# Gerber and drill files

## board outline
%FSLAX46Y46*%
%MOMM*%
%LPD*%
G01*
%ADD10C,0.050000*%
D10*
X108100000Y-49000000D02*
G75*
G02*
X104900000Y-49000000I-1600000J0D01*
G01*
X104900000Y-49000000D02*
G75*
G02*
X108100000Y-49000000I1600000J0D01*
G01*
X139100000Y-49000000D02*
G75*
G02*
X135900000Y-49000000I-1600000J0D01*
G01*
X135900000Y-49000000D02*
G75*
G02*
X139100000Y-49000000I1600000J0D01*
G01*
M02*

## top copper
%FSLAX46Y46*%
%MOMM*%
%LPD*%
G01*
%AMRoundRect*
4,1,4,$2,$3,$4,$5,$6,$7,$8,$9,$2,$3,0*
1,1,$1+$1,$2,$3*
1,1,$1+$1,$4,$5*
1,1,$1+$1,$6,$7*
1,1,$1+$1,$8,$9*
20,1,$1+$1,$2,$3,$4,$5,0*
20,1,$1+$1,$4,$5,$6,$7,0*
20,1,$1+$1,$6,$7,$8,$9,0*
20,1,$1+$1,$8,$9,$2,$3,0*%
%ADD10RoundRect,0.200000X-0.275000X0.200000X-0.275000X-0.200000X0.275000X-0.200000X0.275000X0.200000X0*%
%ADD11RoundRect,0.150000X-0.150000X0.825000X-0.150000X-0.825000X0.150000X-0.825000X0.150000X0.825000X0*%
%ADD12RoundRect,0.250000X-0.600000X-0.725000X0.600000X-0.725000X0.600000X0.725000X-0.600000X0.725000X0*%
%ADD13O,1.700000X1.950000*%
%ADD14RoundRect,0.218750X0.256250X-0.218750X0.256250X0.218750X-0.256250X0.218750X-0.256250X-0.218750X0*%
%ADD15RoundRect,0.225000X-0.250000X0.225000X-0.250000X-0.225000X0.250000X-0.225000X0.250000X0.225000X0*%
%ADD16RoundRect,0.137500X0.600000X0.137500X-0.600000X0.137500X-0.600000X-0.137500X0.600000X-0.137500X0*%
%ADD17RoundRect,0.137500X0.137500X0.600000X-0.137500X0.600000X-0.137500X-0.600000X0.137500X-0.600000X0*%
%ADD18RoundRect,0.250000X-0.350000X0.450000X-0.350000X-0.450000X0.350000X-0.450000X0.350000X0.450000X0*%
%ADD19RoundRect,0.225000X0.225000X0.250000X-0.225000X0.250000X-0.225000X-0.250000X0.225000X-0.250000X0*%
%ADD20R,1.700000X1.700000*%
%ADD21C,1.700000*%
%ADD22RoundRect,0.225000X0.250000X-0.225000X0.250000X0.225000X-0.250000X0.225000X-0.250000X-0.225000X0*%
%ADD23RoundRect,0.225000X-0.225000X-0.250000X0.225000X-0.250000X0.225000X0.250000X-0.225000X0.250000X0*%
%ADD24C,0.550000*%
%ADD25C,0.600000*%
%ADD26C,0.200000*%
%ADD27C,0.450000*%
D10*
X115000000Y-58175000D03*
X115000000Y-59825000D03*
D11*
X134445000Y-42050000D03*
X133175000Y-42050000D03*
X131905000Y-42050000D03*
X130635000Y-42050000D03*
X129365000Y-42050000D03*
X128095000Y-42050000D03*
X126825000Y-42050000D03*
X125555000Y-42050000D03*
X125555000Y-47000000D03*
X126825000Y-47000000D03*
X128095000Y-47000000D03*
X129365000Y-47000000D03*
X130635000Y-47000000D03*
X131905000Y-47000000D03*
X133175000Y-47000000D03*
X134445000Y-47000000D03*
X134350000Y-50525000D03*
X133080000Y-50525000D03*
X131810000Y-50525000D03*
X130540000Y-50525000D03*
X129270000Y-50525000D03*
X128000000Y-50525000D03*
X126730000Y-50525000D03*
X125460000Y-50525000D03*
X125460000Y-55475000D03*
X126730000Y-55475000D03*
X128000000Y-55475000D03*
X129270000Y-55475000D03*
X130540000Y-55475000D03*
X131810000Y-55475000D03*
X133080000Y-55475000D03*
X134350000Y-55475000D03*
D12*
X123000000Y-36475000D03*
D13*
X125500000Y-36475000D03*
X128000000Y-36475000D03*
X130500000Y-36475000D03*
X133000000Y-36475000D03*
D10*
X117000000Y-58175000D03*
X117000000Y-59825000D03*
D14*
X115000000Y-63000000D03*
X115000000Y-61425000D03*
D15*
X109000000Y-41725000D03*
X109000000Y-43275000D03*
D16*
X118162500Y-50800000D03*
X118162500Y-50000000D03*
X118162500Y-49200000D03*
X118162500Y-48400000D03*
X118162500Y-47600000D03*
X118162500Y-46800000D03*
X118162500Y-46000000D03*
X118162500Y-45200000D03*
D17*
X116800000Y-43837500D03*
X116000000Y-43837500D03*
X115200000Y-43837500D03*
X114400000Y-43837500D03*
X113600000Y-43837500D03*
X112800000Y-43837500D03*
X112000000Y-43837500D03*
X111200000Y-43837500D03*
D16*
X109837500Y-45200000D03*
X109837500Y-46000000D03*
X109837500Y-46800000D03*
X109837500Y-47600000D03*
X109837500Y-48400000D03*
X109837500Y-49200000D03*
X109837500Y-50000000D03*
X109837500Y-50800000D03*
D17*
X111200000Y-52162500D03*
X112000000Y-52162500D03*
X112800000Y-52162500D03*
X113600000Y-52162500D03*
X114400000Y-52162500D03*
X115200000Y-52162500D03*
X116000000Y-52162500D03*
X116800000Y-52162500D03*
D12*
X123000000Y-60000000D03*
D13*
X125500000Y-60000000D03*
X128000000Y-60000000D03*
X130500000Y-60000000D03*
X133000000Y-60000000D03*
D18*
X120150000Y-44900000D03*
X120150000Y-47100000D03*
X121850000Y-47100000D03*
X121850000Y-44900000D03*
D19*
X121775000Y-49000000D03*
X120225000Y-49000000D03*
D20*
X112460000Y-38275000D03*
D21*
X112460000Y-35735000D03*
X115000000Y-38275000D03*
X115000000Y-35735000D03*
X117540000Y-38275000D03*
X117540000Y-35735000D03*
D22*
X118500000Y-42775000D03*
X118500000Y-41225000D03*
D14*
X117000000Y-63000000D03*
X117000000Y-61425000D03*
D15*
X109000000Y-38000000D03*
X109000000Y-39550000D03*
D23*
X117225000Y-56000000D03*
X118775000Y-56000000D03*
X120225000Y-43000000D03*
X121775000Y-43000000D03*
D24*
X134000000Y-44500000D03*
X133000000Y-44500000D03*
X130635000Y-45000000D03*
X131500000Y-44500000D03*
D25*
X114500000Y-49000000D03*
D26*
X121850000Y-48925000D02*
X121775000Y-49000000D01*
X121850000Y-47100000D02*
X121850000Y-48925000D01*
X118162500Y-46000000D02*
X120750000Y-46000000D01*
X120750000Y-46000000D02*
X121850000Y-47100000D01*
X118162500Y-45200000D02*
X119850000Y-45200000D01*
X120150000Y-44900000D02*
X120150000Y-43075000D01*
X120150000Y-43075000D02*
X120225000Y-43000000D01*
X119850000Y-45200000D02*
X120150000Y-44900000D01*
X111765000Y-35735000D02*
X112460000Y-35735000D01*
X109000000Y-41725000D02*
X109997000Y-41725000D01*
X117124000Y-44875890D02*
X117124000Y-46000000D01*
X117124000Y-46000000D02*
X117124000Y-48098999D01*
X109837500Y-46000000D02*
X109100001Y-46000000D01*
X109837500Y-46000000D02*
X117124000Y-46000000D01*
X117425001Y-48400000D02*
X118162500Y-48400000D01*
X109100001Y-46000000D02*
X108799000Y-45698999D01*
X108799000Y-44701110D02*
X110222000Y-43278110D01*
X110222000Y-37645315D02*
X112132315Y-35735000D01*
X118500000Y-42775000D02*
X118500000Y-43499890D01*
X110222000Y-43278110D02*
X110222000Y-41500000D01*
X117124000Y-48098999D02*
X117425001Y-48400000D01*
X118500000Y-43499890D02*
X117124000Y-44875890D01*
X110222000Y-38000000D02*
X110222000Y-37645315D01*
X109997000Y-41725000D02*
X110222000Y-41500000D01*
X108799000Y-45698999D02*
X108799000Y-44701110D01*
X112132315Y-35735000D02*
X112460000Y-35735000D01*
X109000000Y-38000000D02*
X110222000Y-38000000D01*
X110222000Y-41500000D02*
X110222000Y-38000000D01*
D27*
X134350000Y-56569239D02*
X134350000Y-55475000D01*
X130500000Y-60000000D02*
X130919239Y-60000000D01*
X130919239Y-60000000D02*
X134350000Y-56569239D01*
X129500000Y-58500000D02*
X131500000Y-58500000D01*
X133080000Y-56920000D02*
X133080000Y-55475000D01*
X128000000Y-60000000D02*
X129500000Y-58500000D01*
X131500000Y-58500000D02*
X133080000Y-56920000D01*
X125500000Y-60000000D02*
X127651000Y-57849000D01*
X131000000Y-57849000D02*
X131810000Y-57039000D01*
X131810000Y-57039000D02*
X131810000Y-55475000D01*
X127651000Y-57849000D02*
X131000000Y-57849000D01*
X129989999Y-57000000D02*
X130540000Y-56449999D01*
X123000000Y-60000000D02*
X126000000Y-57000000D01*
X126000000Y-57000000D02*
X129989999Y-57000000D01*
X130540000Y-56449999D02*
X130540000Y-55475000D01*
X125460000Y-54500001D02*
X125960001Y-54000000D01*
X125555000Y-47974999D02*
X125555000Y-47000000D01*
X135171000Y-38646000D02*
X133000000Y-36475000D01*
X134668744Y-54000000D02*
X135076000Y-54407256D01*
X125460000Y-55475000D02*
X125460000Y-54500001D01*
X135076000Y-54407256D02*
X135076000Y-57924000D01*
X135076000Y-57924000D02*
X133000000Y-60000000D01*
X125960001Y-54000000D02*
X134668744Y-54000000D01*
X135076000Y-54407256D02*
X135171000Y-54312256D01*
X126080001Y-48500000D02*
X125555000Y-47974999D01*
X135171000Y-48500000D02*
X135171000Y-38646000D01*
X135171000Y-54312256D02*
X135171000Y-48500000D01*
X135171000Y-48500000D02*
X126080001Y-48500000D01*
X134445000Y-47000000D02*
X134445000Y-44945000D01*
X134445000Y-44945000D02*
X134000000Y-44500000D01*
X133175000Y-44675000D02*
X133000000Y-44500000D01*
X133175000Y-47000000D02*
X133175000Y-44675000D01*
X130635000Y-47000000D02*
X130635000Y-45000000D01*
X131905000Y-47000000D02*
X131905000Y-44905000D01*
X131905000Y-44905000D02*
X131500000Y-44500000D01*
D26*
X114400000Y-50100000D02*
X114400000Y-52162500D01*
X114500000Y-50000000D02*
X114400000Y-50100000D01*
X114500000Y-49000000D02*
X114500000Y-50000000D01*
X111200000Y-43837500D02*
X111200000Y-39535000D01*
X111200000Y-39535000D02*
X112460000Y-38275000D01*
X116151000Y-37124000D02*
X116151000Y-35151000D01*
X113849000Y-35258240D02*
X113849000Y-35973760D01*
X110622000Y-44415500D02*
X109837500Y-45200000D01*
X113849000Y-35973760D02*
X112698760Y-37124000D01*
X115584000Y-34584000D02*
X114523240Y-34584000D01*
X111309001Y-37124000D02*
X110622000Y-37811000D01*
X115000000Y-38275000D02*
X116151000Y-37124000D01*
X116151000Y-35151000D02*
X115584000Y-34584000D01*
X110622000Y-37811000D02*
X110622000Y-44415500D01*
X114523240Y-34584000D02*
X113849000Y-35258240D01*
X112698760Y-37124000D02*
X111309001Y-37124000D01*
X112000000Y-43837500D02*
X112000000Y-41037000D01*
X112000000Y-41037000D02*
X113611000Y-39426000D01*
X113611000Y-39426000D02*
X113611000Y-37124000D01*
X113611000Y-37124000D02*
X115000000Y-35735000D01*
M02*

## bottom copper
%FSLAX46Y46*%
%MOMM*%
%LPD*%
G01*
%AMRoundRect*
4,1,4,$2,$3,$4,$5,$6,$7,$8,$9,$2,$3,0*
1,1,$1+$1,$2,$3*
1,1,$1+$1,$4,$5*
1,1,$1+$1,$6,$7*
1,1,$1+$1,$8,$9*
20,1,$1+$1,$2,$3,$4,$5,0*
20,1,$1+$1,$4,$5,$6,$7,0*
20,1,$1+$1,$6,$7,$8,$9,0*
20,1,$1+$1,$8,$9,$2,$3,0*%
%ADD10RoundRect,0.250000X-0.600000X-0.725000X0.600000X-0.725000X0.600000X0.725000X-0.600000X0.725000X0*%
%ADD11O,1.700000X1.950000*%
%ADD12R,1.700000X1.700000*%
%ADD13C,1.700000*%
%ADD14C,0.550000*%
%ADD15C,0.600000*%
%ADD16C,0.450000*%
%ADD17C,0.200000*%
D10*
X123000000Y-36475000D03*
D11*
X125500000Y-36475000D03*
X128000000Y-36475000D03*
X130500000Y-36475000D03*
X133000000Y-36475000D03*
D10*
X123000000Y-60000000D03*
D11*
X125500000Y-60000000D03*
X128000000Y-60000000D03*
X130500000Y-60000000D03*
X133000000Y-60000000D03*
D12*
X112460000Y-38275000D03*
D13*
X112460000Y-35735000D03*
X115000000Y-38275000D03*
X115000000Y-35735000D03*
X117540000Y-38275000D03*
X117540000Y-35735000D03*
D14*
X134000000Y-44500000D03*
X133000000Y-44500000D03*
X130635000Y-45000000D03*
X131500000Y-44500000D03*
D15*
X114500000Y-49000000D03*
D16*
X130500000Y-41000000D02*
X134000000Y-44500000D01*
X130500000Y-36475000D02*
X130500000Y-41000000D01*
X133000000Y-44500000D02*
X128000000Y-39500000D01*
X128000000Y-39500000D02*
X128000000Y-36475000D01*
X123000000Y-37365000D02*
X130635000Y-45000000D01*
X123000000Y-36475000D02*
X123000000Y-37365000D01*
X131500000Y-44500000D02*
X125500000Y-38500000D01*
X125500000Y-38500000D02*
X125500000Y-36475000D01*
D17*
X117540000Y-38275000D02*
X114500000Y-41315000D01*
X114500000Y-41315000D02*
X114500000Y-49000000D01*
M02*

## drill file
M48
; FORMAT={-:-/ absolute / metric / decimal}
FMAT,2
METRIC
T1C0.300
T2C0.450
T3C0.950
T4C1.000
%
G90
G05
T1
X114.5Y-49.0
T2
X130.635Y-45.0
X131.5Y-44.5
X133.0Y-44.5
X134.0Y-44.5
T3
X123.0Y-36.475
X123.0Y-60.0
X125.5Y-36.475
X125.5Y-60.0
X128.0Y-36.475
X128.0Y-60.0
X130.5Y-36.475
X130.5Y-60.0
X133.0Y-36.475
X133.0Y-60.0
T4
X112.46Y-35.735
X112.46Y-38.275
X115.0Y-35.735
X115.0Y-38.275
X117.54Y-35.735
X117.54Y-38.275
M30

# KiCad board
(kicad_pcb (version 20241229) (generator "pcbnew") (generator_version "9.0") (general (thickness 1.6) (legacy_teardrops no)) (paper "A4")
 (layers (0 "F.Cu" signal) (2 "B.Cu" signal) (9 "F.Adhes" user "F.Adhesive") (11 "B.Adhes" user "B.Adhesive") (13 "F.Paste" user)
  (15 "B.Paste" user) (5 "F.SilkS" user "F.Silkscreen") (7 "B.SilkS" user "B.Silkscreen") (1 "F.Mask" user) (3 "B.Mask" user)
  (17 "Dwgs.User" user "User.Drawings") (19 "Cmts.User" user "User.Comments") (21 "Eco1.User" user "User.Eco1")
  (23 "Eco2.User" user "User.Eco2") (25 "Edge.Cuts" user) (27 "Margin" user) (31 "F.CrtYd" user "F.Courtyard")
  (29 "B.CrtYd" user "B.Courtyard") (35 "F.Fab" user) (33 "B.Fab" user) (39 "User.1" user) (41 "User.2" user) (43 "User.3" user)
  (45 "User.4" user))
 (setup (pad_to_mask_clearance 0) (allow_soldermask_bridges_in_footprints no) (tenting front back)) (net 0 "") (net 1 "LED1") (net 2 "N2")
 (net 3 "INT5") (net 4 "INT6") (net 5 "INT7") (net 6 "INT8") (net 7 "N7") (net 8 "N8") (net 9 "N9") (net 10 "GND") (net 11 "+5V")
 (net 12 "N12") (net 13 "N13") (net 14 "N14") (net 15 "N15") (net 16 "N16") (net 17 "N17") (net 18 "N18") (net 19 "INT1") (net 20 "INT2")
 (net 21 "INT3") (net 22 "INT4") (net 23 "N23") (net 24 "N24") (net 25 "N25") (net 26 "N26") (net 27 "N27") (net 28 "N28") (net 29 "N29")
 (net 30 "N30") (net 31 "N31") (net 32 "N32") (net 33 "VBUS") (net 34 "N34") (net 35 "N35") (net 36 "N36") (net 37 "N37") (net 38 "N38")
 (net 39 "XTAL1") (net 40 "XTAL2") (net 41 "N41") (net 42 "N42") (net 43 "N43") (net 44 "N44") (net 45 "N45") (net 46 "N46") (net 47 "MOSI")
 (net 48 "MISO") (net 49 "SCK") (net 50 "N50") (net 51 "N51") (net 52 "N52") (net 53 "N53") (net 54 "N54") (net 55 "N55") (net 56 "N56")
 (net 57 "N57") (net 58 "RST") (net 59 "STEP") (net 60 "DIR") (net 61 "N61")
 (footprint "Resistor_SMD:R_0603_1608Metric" (layer "F.Cu") (at 115 59 -90)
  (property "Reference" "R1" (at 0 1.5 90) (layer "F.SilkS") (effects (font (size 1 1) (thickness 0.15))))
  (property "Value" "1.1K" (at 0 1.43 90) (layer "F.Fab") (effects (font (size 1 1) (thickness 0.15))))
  (pad "1" smd roundrect (at -0.825 0 270) (size 0.8 0.95) (layers "F.Cu" "F.Mask" "F.Paste") (roundrect_rratio 0.25) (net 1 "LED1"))
  (pad "2" smd roundrect (at 0.825 0 270) (size 0.8 0.95) (layers "F.Cu" "F.Mask" "F.Paste") (roundrect_rratio 0.25) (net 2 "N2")))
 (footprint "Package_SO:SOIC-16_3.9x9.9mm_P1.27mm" (layer "F.Cu") (at 130 44.525 -90)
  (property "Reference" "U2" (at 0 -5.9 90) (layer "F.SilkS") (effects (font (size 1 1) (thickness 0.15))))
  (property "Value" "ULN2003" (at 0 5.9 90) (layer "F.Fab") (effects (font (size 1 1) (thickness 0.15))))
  (pad "1" smd roundrect (at -2.475 -4.445 270) (size 1.95 0.6) (layers "F.Cu" "F.Mask" "F.Paste") (roundrect_rratio 0.25) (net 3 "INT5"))
  (pad "2" smd roundrect (at -2.475 -3.175 270) (size 1.95 0.6) (layers "F.Cu" "F.Mask" "F.Paste") (roundrect_rratio 0.25) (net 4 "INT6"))
  (pad "3" smd roundrect (at -2.475 -1.905 270) (size 1.95 0.6) (layers "F.Cu" "F.Mask" "F.Paste") (roundrect_rratio 0.25) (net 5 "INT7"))
  (pad "4" smd roundrect (at -2.475 -0.635 270) (size 1.95 0.6) (layers "F.Cu" "F.Mask" "F.Paste") (roundrect_rratio 0.25) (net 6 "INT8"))
  (pad "5" smd roundrect (at -2.475 0.635 270) (size 1.95 0.6) (layers "F.Cu" "F.Mask" "F.Paste") (roundrect_rratio 0.25) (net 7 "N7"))
  (pad "6" smd roundrect (at -2.475 1.905 270) (size 1.95 0.6) (layers "F.Cu" "F.Mask" "F.Paste") (roundrect_rratio 0.25) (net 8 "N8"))
  (pad "7" smd roundrect (at -2.475 3.175 270) (size 1.95 0.6) (layers "F.Cu" "F.Mask" "F.Paste") (roundrect_rratio 0.25) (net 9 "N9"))
  (pad "8" smd roundrect (at -2.475 4.445 270) (size 1.95 0.6) (layers "F.Cu" "F.Mask" "F.Paste") (roundrect_rratio 0.25) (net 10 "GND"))
  (pad "9" smd roundrect (at 2.475 4.445 270) (size 1.95 0.6) (layers "F.Cu" "F.Mask" "F.Paste") (roundrect_rratio 0.25) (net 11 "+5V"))
  (pad "10" smd roundrect (at 2.475 3.175 270) (size 1.95 0.6) (layers "F.Cu" "F.Mask" "F.Paste") (roundrect_rratio 0.25) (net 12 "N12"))
  (pad "11" smd roundrect (at 2.475 1.905 270) (size 1.95 0.6) (layers "F.Cu" "F.Mask" "F.Paste") (roundrect_rratio 0.25) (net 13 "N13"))
  (pad "12" smd roundrect (at 2.475 0.635 270) (size 1.95 0.6) (layers "F.Cu" "F.Mask" "F.Paste") (roundrect_rratio 0.25) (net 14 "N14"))
  (pad "13" smd roundrect (at 2.475 -0.635 270) (size 1.95 0.6) (layers "F.Cu" "F.Mask" "F.Paste") (roundrect_rratio 0.25) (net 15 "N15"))
  (pad "14" smd roundrect (at 2.475 -1.905 270) (size 1.95 0.6) (layers "F.Cu" "F.Mask" "F.Paste") (roundrect_rratio 0.25) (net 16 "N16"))
  (pad "15" smd roundrect (at 2.475 -3.175 270) (size 1.95 0.6) (layers "F.Cu" "F.Mask" "F.Paste") (roundrect_rratio 0.25) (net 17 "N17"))
  (pad "16" smd roundrect (at 2.475 -4.445 270) (size 1.95 0.6) (layers "F.Cu" "F.Mask" "F.Paste") (roundrect_rratio 0.25) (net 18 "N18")))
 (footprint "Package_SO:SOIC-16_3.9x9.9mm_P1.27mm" (layer "F.Cu") (at 129.905 53 -90)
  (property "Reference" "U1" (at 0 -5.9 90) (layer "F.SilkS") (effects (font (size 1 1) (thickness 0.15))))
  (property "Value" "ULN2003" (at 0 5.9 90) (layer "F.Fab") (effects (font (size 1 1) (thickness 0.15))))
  (pad "1" smd roundrect (at -2.475 -4.445 270) (size 1.95 0.6) (layers "F.Cu" "F.Mask" "F.Paste") (roundrect_rratio 0.25) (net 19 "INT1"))
  (pad "2" smd roundrect (at -2.475 -3.175 270) (size 1.95 0.6) (layers "F.Cu" "F.Mask" "F.Paste") (roundrect_rratio 0.25) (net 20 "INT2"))
  (pad "3" smd roundrect (at -2.475 -1.905 270) (size 1.95 0.6) (layers "F.Cu" "F.Mask" "F.Paste") (roundrect_rratio 0.25) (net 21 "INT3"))
  (pad "4" smd roundrect (at -2.475 -0.635 270) (size 1.95 0.6) (layers "F.Cu" "F.Mask" "F.Paste") (roundrect_rratio 0.25) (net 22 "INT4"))
  (pad "5" smd roundrect (at -2.475 0.635 270) (size 1.95 0.6) (layers "F.Cu" "F.Mask" "F.Paste") (roundrect_rratio 0.25) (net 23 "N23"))
  (pad "6" smd roundrect (at -2.475 1.905 270) (size 1.95 0.6) (layers "F.Cu" "F.Mask" "F.Paste") (roundrect_rratio 0.25) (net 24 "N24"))
  (pad "7" smd roundrect (at -2.475 3.175 270) (size 1.95 0.6) (layers "F.Cu" "F.Mask" "F.Paste") (roundrect_rratio 0.25) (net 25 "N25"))
  (pad "8" smd roundrect (at -2.475 4.445 270) (size 1.95 0.6) (layers "F.Cu" "F.Mask" "F.Paste") (roundrect_rratio 0.25) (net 10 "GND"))
  (pad "9" smd roundrect (at 2.475 4.445 270) (size 1.95 0.6) (layers "F.Cu" "F.Mask" "F.Paste") (roundrect_rratio 0.25) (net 11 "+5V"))
  (pad "10" smd roundrect (at 2.475 3.175 270) (size 1.95 0.6) (layers "F.Cu" "F.Mask" "F.Paste") (roundrect_rratio 0.25) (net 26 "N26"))
  (pad "11" smd roundrect (at 2.475 1.905 270) (size 1.95 0.6) (layers "F.Cu" "F.Mask" "F.Paste") (roundrect_rratio 0.25) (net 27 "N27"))
  (pad "12" smd roundrect (at 2.475 0.635 270) (size 1.95 0.6) (layers "F.Cu" "F.Mask" "F.Paste") (roundrect_rratio 0.25) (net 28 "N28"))
  (pad "13" smd roundrect (at 2.475 -0.635 270) (size 1.95 0.6) (layers "F.Cu" "F.Mask" "F.Paste") (roundrect_rratio 0.25) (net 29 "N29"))
  (pad "14" smd roundrect (at 2.475 -1.905 270) (size 1.95 0.6) (layers "F.Cu" "F.Mask" "F.Paste") (roundrect_rratio 0.25) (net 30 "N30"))
  (pad "15" smd roundrect (at 2.475 -3.175 270) (size 1.95 0.6) (layers "F.Cu" "F.Mask" "F.Paste") (roundrect_rratio 0.25) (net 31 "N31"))
  (pad "16" smd roundrect (at 2.475 -4.445 270) (size 1.95 0.6) (layers "F.Cu" "F.Mask" "F.Paste") (roundrect_rratio 0.25) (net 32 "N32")))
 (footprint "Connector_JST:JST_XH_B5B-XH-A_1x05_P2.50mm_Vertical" (layer "F.Cu") (at 123 36.475)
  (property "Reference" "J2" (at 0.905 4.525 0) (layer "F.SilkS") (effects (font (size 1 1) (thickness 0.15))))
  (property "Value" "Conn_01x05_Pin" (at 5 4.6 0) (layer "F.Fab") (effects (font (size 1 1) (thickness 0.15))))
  (pad "1" thru_hole roundrect (at 0 0) (size 1.7 1.95) (drill 0.95) (layers "*.Cu" "*.Mask") (remove_unused_layers no)
   (roundrect_rratio 0.147059) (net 15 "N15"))
  (pad "2" thru_hole oval (at 2.5 0) (size 1.7 1.95) (drill 0.95) (layers "*.Cu" "*.Mask") (remove_unused_layers no) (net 16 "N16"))
  (pad "3" thru_hole oval (at 5 0) (size 1.7 1.95) (drill 0.95) (layers "*.Cu" "*.Mask") (remove_unused_layers no) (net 17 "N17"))
  (pad "4" thru_hole oval (at 7.5 0) (size 1.7 1.95) (drill 0.95) (layers "*.Cu" "*.Mask") (remove_unused_layers no) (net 18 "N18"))
  (pad "5" thru_hole oval (at 10 0) (size 1.7 1.95) (drill 0.95) (layers "*.Cu" "*.Mask") (remove_unused_layers no) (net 11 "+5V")))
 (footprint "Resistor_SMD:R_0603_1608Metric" (layer "F.Cu") (at 117 59 -90)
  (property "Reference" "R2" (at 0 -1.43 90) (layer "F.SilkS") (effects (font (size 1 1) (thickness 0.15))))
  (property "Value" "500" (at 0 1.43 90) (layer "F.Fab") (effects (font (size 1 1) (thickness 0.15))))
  (pad "1" smd roundrect (at -0.825 0 270) (size 0.8 0.95) (layers "F.Cu" "F.Mask" "F.Paste") (roundrect_rratio 0.25) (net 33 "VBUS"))
  (pad "2" smd roundrect (at 0.825 0 270) (size 0.8 0.95) (layers "F.Cu" "F.Mask" "F.Paste") (roundrect_rratio 0.25) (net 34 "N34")))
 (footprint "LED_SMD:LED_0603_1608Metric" (layer "F.Cu") (at 115 62.2125 90)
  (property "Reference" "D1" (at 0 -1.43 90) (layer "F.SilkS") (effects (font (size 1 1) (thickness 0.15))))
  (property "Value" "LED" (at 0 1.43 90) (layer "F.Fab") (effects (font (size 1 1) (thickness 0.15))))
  (pad "1" smd roundrect (at -0.7875 0 90) (size 0.875 0.95) (layers "F.Cu" "F.Mask" "F.Paste") (roundrect_rratio 0.25) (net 10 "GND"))
  (pad "2" smd roundrect (at 0.7875 0 90) (size 0.875 0.95) (layers "F.Cu" "F.Mask" "F.Paste") (roundrect_rratio 0.25) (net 2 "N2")))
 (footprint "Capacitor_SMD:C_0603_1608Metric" (layer "F.Cu") (at 109 42.5 -90)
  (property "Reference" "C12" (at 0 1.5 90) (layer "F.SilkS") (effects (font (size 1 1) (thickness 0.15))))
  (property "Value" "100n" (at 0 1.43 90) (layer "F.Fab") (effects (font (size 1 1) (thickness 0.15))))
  (pad "1" smd roundrect (at -0.775 0 270) (size 0.9 0.95) (layers "F.Cu" "F.Mask" "F.Paste") (roundrect_rratio 0.25) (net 33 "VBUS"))
  (pad "2" smd roundrect (at 0.775 0 270) (size 0.9 0.95) (layers "F.Cu" "F.Mask" "F.Paste") (roundrect_rratio 0.25) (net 10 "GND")))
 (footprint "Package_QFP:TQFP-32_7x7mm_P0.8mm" (layer "F.Cu") (at 114 48 180)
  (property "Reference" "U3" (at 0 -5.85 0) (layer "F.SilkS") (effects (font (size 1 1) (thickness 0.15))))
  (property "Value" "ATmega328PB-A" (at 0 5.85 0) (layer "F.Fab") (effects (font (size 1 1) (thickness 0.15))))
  (pad "1" smd roundrect (at -4.1625 -2.8 180) (size 1.475 0.55) (layers "F.Cu" "F.Mask" "F.Paste") (roundrect_rratio 0.25) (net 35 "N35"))
  (pad "2" smd roundrect (at -4.1625 -2 180) (size 1.475 0.55) (layers "F.Cu" "F.Mask" "F.Paste") (roundrect_rratio 0.25) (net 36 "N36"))
  (pad "3" smd roundrect (at -4.1625 -1.2 180) (size 1.475 0.55) (layers "F.Cu" "F.Mask" "F.Paste") (roundrect_rratio 0.25) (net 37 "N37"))
  (pad "4" smd roundrect (at -4.1625 -0.4 180) (size 1.475 0.55) (layers "F.Cu" "F.Mask" "F.Paste") (roundrect_rratio 0.25) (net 33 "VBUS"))
  (pad "5" smd roundrect (at -4.1625 0.4 180) (size 1.475 0.55) (layers "F.Cu" "F.Mask" "F.Paste") (roundrect_rratio 0.25) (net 10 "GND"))
  (pad "6" smd roundrect (at -4.1625 1.2 180) (size 1.475 0.55) (layers "F.Cu" "F.Mask" "F.Paste") (roundrect_rratio 0.25) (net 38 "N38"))
  (pad "7" smd roundrect (at -4.1625 2 180) (size 1.475 0.55) (layers "F.Cu" "F.Mask" "F.Paste") (roundrect_rratio 0.25) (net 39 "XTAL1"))
  (pad "8" smd roundrect (at -4.1625 2.8 180) (size 1.475 0.55) (layers "F.Cu" "F.Mask" "F.Paste") (roundrect_rratio 0.25) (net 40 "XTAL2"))
  (pad "9" smd roundrect (at -2.8 4.1625 180) (size 0.55 1.475) (layers "F.Cu" "F.Mask" "F.Paste") (roundrect_rratio 0.25) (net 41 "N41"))
  (pad "10" smd roundrect (at -2 4.1625 180) (size 0.55 1.475) (layers "F.Cu" "F.Mask" "F.Paste") (roundrect_rratio 0.25) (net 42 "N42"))
  (pad "11" smd roundrect (at -1.2 4.1625 180) (size 0.55 1.475) (layers "F.Cu" "F.Mask" "F.Paste") (roundrect_rratio 0.25) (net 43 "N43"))
  (pad "12" smd roundrect (at -0.4 4.1625 180) (size 0.55 1.475) (layers "F.Cu" "F.Mask" "F.Paste") (roundrect_rratio 0.25) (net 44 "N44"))
  (pad "13" smd roundrect (at 0.4 4.1625 180) (size 0.55 1.475) (layers "F.Cu" "F.Mask" "F.Paste") (roundrect_rratio 0.25) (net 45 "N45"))
  (pad "14" smd roundrect (at 1.2 4.1625 180) (size 0.55 1.475) (layers "F.Cu" "F.Mask" "F.Paste") (roundrect_rratio 0.25) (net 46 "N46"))
  (pad "15" smd roundrect (at 2 4.1625 180) (size 0.55 1.475) (layers "F.Cu" "F.Mask" "F.Paste") (roundrect_rratio 0.25) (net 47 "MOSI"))
  (pad "16" smd roundrect (at 2.8 4.1625 180) (size 0.55 1.475) (layers "F.Cu" "F.Mask" "F.Paste") (roundrect_rratio 0.25) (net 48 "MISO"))
  (pad "17" smd roundrect (at 4.1625 2.8 180) (size 1.475 0.55) (layers "F.Cu" "F.Mask" "F.Paste") (roundrect_rratio 0.25) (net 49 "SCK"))
  (pad "18" smd roundrect (at 4.1625 2 180) (size 1.475 0.55) (layers "F.Cu" "F.Mask" "F.Paste") (roundrect_rratio 0.25) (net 33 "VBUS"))
  (pad "19" smd roundrect (at 4.1625 1.2 180) (size 1.475 0.55) (layers "F.Cu" "F.Mask" "F.Paste") (roundrect_rratio 0.25) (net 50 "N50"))
  (pad "20" smd roundrect (at 4.1625 0.4 180) (size 1.475 0.55) (layers "F.Cu" "F.Mask" "F.Paste") (roundrect_rratio 0.25) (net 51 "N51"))
  (pad "21" smd roundrect (at 4.1625 -0.4 180) (size 1.475 0.55) (layers "F.Cu" "F.Mask" "F.Paste") (roundrect_rratio 0.25) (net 10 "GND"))
  (pad "22" smd roundrect (at 4.1625 -1.2 180) (size 1.475 0.55) (layers "F.Cu" "F.Mask" "F.Paste") (roundrect_rratio 0.25) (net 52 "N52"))
  (pad "23" smd roundrect (at 4.1625 -2 180) (size 1.475 0.55) (layers "F.Cu" "F.Mask" "F.Paste") (roundrect_rratio 0.25) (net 1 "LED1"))
  (pad "24" smd roundrect (at 4.1625 -2.8 180) (size 1.475 0.55) (layers "F.Cu" "F.Mask" "F.Paste") (roundrect_rratio 0.25) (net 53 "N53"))
  (pad "25" smd roundrect (at 2.8 -4.1625 180) (size 0.55 1.475) (layers "F.Cu" "F.Mask" "F.Paste") (roundrect_rratio 0.25) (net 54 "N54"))
  (pad "26" smd roundrect (at 2 -4.1625 180) (size 0.55 1.475) (layers "F.Cu" "F.Mask" "F.Paste") (roundrect_rratio 0.25) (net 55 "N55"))
  (pad "27" smd roundrect (at 1.2 -4.1625 180) (size 0.55 1.475) (layers "F.Cu" "F.Mask" "F.Paste") (roundrect_rratio 0.25) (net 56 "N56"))
  (pad "28" smd roundrect (at 0.4 -4.1625 180) (size 0.55 1.475) (layers "F.Cu" "F.Mask" "F.Paste") (roundrect_rratio 0.25) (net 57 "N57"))
  (pad "29" smd roundrect (at -0.4 -4.1625 180) (size 0.55 1.475) (layers "F.Cu" "F.Mask" "F.Paste") (roundrect_rratio 0.25) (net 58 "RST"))
  (pad "30" smd roundrect (at -1.2 -4.1625 180) (size 0.55 1.475) (layers "F.Cu" "F.Mask" "F.Paste") (roundrect_rratio 0.25) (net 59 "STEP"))
  (pad "31" smd roundrect (at -2 -4.1625 180) (size 0.55 1.475) (layers "F.Cu" "F.Mask" "F.Paste") (roundrect_rratio 0.25) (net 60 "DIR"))
  (pad "32" smd roundrect (at -2.8 -4.1625 180) (size 0.55 1.475) (layers "F.Cu" "F.Mask" "F.Paste") (roundrect_rratio 0.25) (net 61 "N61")))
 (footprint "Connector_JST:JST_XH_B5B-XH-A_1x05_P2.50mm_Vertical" (layer "F.Cu") (at 123 60)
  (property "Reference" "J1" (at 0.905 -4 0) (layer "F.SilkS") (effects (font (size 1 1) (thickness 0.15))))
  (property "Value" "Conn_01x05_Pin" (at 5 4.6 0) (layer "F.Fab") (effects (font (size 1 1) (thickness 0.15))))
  (pad "1" thru_hole roundrect (at 0 0) (size 1.7 1.95) (drill 0.95) (layers "*.Cu" "*.Mask") (remove_unused_layers no)
   (roundrect_rratio 0.147059) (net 29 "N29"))
  (pad "2" thru_hole oval (at 2.5 0) (size 1.7 1.95) (drill 0.95) (layers "*.Cu" "*.Mask") (remove_unused_layers no) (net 30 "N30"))
  (pad "3" thru_hole oval (at 5 0) (size 1.7 1.95) (drill 0.95) (layers "*.Cu" "*.Mask") (remove_unused_layers no) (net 31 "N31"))
  (pad "4" thru_hole oval (at 7.5 0) (size 1.7 1.95) (drill 0.95) (layers "*.Cu" "*.Mask") (remove_unused_layers no) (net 32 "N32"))
  (pad "5" thru_hole oval (at 10 0) (size 1.7 1.95) (drill 0.95) (layers "*.Cu" "*.Mask") (remove_unused_layers no) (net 11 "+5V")))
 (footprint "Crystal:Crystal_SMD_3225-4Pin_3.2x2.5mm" (layer "F.Cu") (at 121 46 -90)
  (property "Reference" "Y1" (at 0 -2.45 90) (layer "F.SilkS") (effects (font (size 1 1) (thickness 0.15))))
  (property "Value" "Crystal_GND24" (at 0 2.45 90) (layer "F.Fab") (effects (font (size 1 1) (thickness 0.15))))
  (pad "1" smd roundrect (at -1.1 0.85 270) (size 1.4 1.2) (layers "F.Cu" "F.Mask" "F.Paste") (roundrect_rratio 0.208333) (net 40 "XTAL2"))
  (pad "2" smd roundrect (at 1.1 0.85 270) (size 1.4 1.2) (layers "F.Cu" "F.Mask" "F.Paste") (roundrect_rratio 0.208333) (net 10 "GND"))
  (pad "3" smd roundrect (at 1.1 -0.85 270) (size 1.4 1.2) (layers "F.Cu" "F.Mask" "F.Paste") (roundrect_rratio 0.208333) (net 39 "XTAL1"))
  (pad "4" smd roundrect (at -1.1 -0.85 270) (size 1.4 1.2) (layers "F.Cu" "F.Mask" "F.Paste") (roundrect_rratio 0.208333) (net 10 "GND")))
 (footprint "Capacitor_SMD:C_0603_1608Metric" (layer "F.Cu") (at 121 49 180)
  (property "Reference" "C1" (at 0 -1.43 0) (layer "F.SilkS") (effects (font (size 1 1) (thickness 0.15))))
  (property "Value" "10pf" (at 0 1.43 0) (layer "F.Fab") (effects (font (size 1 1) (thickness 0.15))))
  (pad "1" smd roundrect (at -0.775 0 180) (size 0.9 0.95) (layers "F.Cu" "F.Mask" "F.Paste") (roundrect_rratio 0.25) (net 39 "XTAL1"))
  (pad "2" smd roundrect (at 0.775 0 180) (size 0.9 0.95) (layers "F.Cu" "F.Mask" "F.Paste") (roundrect_rratio 0.25) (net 10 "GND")))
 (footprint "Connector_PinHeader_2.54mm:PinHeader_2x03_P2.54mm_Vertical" (layer "F.Cu") (at 112.46 38.275 90)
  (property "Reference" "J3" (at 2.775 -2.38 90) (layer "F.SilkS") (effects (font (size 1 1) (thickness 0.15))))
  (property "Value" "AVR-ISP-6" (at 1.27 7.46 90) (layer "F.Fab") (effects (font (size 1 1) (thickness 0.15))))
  (pad "1" thru_hole rect (at 0 0 90) (size 1.7 1.7) (drill 1) (layers "*.Cu" "*.Mask") (remove_unused_layers no) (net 48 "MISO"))
  (pad "2" thru_hole circle (at 2.54 0 90) (size 1.7 1.7) (drill 1) (layers "*.Cu" "*.Mask") (remove_unused_layers no) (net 33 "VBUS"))
  (pad "3" thru_hole circle (at 0 2.54 90) (size 1.7 1.7) (drill 1) (layers "*.Cu" "*.Mask") (remove_unused_layers no) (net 49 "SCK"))
  (pad "4" thru_hole circle (at 2.54 2.54 90) (size 1.7 1.7) (drill 1) (layers "*.Cu" "*.Mask") (remove_unused_layers no) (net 47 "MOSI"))
  (pad "5" thru_hole circle (at 0 5.08 90) (size 1.7 1.7) (drill 1) (layers "*.Cu" "*.Mask") (remove_unused_layers no) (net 58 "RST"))
  (pad "6" thru_hole circle (at 2.54 5.08 90) (size 1.7 1.7) (drill 1) (layers "*.Cu" "*.Mask") (remove_unused_layers no) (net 10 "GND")))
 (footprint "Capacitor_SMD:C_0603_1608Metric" (layer "F.Cu") (at 118.5 42 90)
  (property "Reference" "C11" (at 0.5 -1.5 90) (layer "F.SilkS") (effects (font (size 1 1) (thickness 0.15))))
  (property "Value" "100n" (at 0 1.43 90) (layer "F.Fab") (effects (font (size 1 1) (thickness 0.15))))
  (pad "1" smd roundrect (at -0.775 0 90) (size 0.9 0.95) (layers "F.Cu" "F.Mask" "F.Paste") (roundrect_rratio 0.25) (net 33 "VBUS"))
  (pad "2" smd roundrect (at 0.775 0 90) (size 0.9 0.95) (layers "F.Cu" "F.Mask" "F.Paste") (roundrect_rratio 0.25) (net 10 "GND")))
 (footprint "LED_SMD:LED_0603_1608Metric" (layer "F.Cu") (at 117 62.2125 90)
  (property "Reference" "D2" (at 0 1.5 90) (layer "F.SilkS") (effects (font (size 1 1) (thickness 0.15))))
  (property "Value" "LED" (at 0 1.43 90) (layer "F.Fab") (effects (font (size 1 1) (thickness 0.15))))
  (pad "1" smd roundrect (at -0.7875 0 90) (size 0.875 0.95) (layers "F.Cu" "F.Mask" "F.Paste") (roundrect_rratio 0.25) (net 10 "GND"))
  (pad "2" smd roundrect (at 0.7875 0 90) (size 0.875 0.95) (layers "F.Cu" "F.Mask" "F.Paste") (roundrect_rratio 0.25) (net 34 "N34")))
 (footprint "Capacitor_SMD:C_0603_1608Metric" (layer "F.Cu") (at 109 38.775 -90)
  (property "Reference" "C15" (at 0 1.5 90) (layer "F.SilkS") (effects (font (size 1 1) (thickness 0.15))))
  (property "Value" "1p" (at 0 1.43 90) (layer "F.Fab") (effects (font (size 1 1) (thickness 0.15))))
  (pad "1" smd roundrect (at -0.775 0 270) (size 0.9 0.95) (layers "F.Cu" "F.Mask" "F.Paste") (roundrect_rratio 0.25) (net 33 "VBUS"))
  (pad "2" smd roundrect (at 0.775 0 270) (size 0.9 0.95) (layers "F.Cu" "F.Mask" "F.Paste") (roundrect_rratio 0.25) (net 10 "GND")))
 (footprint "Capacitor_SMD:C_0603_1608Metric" (layer "F.Cu") (at 118 56)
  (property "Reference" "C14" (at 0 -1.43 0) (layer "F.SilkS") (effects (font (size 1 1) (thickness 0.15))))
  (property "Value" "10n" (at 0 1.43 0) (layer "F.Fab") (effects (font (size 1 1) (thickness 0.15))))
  (pad "1" smd roundrect (at -0.775 0) (size 0.9 0.95) (layers "F.Cu" "F.Mask" "F.Paste") (roundrect_rratio 0.25) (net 33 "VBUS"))
  (pad "2" smd roundrect (at 0.775 0) (size 0.9 0.95) (layers "F.Cu" "F.Mask" "F.Paste") (roundrect_rratio 0.25) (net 10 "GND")))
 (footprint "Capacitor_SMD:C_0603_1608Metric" (layer "F.Cu") (at 121 43)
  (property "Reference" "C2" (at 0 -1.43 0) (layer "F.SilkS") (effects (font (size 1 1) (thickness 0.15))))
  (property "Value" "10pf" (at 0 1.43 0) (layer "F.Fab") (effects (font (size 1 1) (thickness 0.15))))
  (pad "1" smd roundrect (at -0.775 0) (size 0.9 0.95) (layers "F.Cu" "F.Mask" "F.Paste") (roundrect_rratio 0.25) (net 40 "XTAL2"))
  (pad "2" smd roundrect (at 0.775 0) (size 0.9 0.95) (layers "F.Cu" "F.Mask" "F.Paste") (roundrect_rratio 0.25) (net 10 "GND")))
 (gr_circle (center 106.5 49) (end 108.1 49) (stroke (width 0.05) (type solid)) (fill no) (layer "Edge.Cuts"))
 (gr_circle (center 137.5 49) (end 139.1 49) (stroke (width 0.05) (type solid)) (fill no) (layer "Edge.Cuts"))
 (segment (start 121.85 48.925) (end 121.775 49) (width 0.2) (layer "F.Cu") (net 39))
 (segment (start 121.85 47.1) (end 121.85 48.925) (width 0.2) (layer "F.Cu") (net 39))
 (segment (start 118.1625 46) (end 120.75 46) (width 0.2) (layer "F.Cu") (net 39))
 (segment (start 120.75 46) (end 121.85 47.1) (width 0.2) (layer "F.Cu") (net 39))
 (segment (start 118.1625 45.2) (end 119.85 45.2) (width 0.2) (layer "F.Cu") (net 40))
 (segment (start 120.15 44.9) (end 120.15 43.075) (width 0.2) (layer "F.Cu") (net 40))
 (segment (start 120.15 43.075) (end 120.225 43) (width 0.2) (layer "F.Cu") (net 40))
 (segment (start 119.85 45.2) (end 120.15 44.9) (width 0.2) (layer "F.Cu") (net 40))
 (segment (start 111.765 35.735) (end 112.46 35.735) (width 0.2) (layer "F.Cu") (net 33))
 (segment (start 109 41.725) (end 109.997 41.725) (width 0.2) (layer "F.Cu") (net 33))
 (segment (start 117.124 44.87589) (end 117.124 46) (width 0.2) (layer "F.Cu") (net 33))
 (segment (start 117.124 46) (end 117.124 48.098999) (width 0.2) (layer "F.Cu") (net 33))
 (segment (start 109.8375 46) (end 109.100001 46) (width 0.2) (layer "F.Cu") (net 33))
 (segment (start 109.8375 46) (end 117.124 46) (width 0.2) (layer "F.Cu") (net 33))
 (segment (start 117.425001 48.4) (end 118.1625 48.4) (width 0.2) (layer "F.Cu") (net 33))
 (segment (start 109.100001 46) (end 108.799 45.698999) (width 0.2) (layer "F.Cu") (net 33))
 (segment (start 108.799 44.70111) (end 110.222 43.27811) (width 0.2) (layer "F.Cu") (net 33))
 (segment (start 110.222 37.645315) (end 112.132315 35.735) (width 0.2) (layer "F.Cu") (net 33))
 (segment (start 118.5 42.775) (end 118.5 43.49989) (width 0.2) (layer "F.Cu") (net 33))
 (segment (start 110.222 43.27811) (end 110.222 41.5) (width 0.2) (layer "F.Cu") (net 33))
 (segment (start 117.124 48.098999) (end 117.425001 48.4) (width 0.2) (layer "F.Cu") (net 33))
 (segment (start 118.5 43.49989) (end 117.124 44.87589) (width 0.2) (layer "F.Cu") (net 33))
 (segment (start 110.222 38) (end 110.222 37.645315) (width 0.2) (layer "F.Cu") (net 33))
 (segment (start 109.997 41.725) (end 110.222 41.5) (width 0.2) (layer "F.Cu") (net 33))
 (segment (start 108.799 45.698999) (end 108.799 44.70111) (width 0.2) (layer "F.Cu") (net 33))
 (segment (start 112.132315 35.735) (end 112.46 35.735) (width 0.2) (layer "F.Cu") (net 33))
 (segment (start 109 38) (end 110.222 38) (width 0.2) (layer "F.Cu") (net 33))
 (segment (start 110.222 41.5) (end 110.222 38) (width 0.2) (layer "F.Cu") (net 33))
 (segment (start 134.35 56.569239) (end 134.35 55.475) (width 0.45) (layer "F.Cu") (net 32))
 (segment (start 130.5 60) (end 130.919239 60) (width 0.45) (layer "F.Cu") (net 32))
 (segment (start 130.919239 60) (end 134.35 56.569239) (width 0.45) (layer "F.Cu") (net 32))
 (segment (start 129.5 58.5) (end 131.5 58.5) (width 0.45) (layer "F.Cu") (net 31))
 (segment (start 133.08 56.92) (end 133.08 55.475) (width 0.45) (layer "F.Cu") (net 31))
 (segment (start 128 60) (end 129.5 58.5) (width 0.45) (layer "F.Cu") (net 31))
 (segment (start 131.5 58.5) (end 133.08 56.92) (width 0.45) (layer "F.Cu") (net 31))
 (segment (start 125.5 60) (end 127.651 57.849) (width 0.45) (layer "F.Cu") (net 30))
 (segment (start 131 57.849) (end 131.81 57.039) (width 0.45) (layer "F.Cu") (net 30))
 (segment (start 131.81 57.039) (end 131.81 55.475) (width 0.45) (layer "F.Cu") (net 30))
 (segment (start 127.651 57.849) (end 131 57.849) (width 0.45) (layer "F.Cu") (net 30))
 (segment (start 129.989999 57) (end 130.54 56.449999) (width 0.45) (layer "F.Cu") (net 29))
 (segment (start 123 60) (end 126 57) (width 0.45) (layer "F.Cu") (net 29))
 (segment (start 126 57) (end 129.989999 57) (width 0.45) (layer "F.Cu") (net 29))
 (segment (start 130.54 56.449999) (end 130.54 55.475) (width 0.45) (layer "F.Cu") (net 29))
 (segment (start 125.46 54.500001) (end 125.960001 54) (width 0.45) (layer "F.Cu") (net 11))
 (segment (start 125.555 47.974999) (end 125.555 47) (width 0.45) (layer "F.Cu") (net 11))
 (segment (start 135.171 38.646) (end 133 36.475) (width 0.45) (layer "F.Cu") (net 11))
 (segment (start 134.668744 54) (end 135.076 54.407256) (width 0.45) (layer "F.Cu") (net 11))
 (segment (start 125.46 55.475) (end 125.46 54.500001) (width 0.45) (layer "F.Cu") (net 11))
 (segment (start 135.076 54.407256) (end 135.076 57.924) (width 0.45) (layer "F.Cu") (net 11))
 (segment (start 135.076 57.924) (end 133 60) (width 0.45) (layer "F.Cu") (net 11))
 (segment (start 125.960001 54) (end 134.668744 54) (width 0.45) (layer "F.Cu") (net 11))
 (segment (start 135.076 54.407256) (end 135.171 54.312256) (width 0.45) (layer "F.Cu") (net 11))
 (segment (start 126.080001 48.5) (end 125.555 47.974999) (width 0.45) (layer "F.Cu") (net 11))
 (segment (start 135.171 48.5) (end 135.171 38.646) (width 0.45) (layer "F.Cu") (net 11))
 (segment (start 135.171 54.312256) (end 135.171 48.5) (width 0.45) (layer "F.Cu") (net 11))
 (segment (start 135.171 48.5) (end 126.080001 48.5) (width 0.45) (layer "F.Cu") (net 11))
 (segment (start 134.445 47) (end 134.445 44.945) (width 0.45) (layer "F.Cu") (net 18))
 (segment (start 134.445 44.945) (end 134 44.5) (width 0.45) (layer "F.Cu") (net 18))
 (via (at 134 44.5) (size 0.55) (drill 0.45) (layers "F.Cu" "B.Cu") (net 18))
 (segment (start 130.5 41) (end 134 44.5) (width 0.45) (layer "B.Cu") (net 18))
 (segment (start 130.5 36.475) (end 130.5 41) (width 0.45) (layer "B.Cu") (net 18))
 (segment (start 133.175 44.675) (end 133 44.5) (width 0.45) (layer "F.Cu") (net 17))
 (segment (start 133.175 47) (end 133.175 44.675) (width 0.45) (layer "F.Cu") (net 17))
 (via (at 133 44.5) (size 0.55) (drill 0.45) (layers "F.Cu" "B.Cu") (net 17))
 (segment (start 133 44.5) (end 128 39.5) (width 0.45) (layer "B.Cu") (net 17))
 (segment (start 128 39.5) (end 128 36.475) (width 0.45) (layer "B.Cu") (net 17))
 (segment (start 130.635 47) (end 130.635 45) (width 0.45) (layer "F.Cu") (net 15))
 (via (at 130.635 45) (size 0.55) (drill 0.45) (layers "F.Cu" "B.Cu") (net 15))
 (segment (start 123 37.365) (end 130.635 45) (width 0.45) (layer "B.Cu") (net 15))
 (segment (start 123 36.475) (end 123 37.365) (width 0.45) (layer "B.Cu") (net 15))
 (segment (start 131.905 47) (end 131.905 44.905) (width 0.45) (layer "F.Cu") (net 16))
 (segment (start 131.905 44.905) (end 131.5 44.5) (width 0.45) (layer "F.Cu") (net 16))
 (via (at 131.5 44.5) (size 0.55) (drill 0.45) (layers "F.Cu" "B.Cu") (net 16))
 (segment (start 131.5 44.5) (end 125.5 38.5) (width 0.45) (layer "B.Cu") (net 16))
 (segment (start 125.5 38.5) (end 125.5 36.475) (width 0.45) (layer "B.Cu") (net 16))
 (segment (start 114.4 50.1) (end 114.4 52.1625) (width 0.2) (layer "F.Cu") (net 58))
 (segment (start 114.5 50) (end 114.4 50.1) (width 0.2) (layer "F.Cu") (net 58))
 (segment (start 114.5 49) (end 114.5 50) (width 0.2) (layer "F.Cu") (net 58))
 (via (at 114.5 49) (size 0.6) (drill 0.3) (layers "F.Cu" "B.Cu") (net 58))
 (segment (start 117.54 38.275) (end 114.5 41.315) (width 0.2) (layer "B.Cu") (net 58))
 (segment (start 114.5 41.315) (end 114.5 49) (width 0.2) (layer "B.Cu") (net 58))
 (segment (start 111.2 43.8375) (end 111.2 39.535) (width 0.2) (layer "F.Cu") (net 48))
 (segment (start 111.2 39.535) (end 112.46 38.275) (width 0.2) (layer "F.Cu") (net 48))
 (segment (start 116.151 37.124) (end 116.151 35.151) (width 0.2) (layer "F.Cu") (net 49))
 (segment (start 113.849 35.25824) (end 113.849 35.97376) (width 0.2) (layer "F.Cu") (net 49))
 (segment (start 110.622 44.4155) (end 109.8375 45.2) (width 0.2) (layer "F.Cu") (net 49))
 (segment (start 113.849 35.97376) (end 112.69876 37.124) (width 0.2) (layer "F.Cu") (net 49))
 (segment (start 115.584 34.584) (end 114.52324 34.584) (width 0.2) (layer "F.Cu") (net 49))
 (segment (start 111.309001 37.124) (end 110.622 37.811) (width 0.2) (layer "F.Cu") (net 49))
 (segment (start 115 38.275) (end 116.151 37.124) (width 0.2) (layer "F.Cu") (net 49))
 (segment (start 116.151 35.151) (end 115.584 34.584) (width 0.2) (layer "F.Cu") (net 49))
 (segment (start 110.622 37.811) (end 110.622 44.4155) (width 0.2) (layer "F.Cu") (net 49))
 (segment (start 114.52324 34.584) (end 113.849 35.25824) (width 0.2) (layer "F.Cu") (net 49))
 (segment (start 112.69876 37.124) (end 111.309001 37.124) (width 0.2) (layer "F.Cu") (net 49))
 (segment (start 112 43.8375) (end 112 41.037) (width 0.2) (layer "F.Cu") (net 47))
 (segment (start 112 41.037) (end 113.611 39.426) (width 0.2) (layer "F.Cu") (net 47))
 (segment (start 113.611 39.426) (end 113.611 37.124) (width 0.2) (layer "F.Cu") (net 47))
 (segment (start 113.611 37.124) (end 115 35.735) (width 0.2) (layer "F.Cu") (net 47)))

